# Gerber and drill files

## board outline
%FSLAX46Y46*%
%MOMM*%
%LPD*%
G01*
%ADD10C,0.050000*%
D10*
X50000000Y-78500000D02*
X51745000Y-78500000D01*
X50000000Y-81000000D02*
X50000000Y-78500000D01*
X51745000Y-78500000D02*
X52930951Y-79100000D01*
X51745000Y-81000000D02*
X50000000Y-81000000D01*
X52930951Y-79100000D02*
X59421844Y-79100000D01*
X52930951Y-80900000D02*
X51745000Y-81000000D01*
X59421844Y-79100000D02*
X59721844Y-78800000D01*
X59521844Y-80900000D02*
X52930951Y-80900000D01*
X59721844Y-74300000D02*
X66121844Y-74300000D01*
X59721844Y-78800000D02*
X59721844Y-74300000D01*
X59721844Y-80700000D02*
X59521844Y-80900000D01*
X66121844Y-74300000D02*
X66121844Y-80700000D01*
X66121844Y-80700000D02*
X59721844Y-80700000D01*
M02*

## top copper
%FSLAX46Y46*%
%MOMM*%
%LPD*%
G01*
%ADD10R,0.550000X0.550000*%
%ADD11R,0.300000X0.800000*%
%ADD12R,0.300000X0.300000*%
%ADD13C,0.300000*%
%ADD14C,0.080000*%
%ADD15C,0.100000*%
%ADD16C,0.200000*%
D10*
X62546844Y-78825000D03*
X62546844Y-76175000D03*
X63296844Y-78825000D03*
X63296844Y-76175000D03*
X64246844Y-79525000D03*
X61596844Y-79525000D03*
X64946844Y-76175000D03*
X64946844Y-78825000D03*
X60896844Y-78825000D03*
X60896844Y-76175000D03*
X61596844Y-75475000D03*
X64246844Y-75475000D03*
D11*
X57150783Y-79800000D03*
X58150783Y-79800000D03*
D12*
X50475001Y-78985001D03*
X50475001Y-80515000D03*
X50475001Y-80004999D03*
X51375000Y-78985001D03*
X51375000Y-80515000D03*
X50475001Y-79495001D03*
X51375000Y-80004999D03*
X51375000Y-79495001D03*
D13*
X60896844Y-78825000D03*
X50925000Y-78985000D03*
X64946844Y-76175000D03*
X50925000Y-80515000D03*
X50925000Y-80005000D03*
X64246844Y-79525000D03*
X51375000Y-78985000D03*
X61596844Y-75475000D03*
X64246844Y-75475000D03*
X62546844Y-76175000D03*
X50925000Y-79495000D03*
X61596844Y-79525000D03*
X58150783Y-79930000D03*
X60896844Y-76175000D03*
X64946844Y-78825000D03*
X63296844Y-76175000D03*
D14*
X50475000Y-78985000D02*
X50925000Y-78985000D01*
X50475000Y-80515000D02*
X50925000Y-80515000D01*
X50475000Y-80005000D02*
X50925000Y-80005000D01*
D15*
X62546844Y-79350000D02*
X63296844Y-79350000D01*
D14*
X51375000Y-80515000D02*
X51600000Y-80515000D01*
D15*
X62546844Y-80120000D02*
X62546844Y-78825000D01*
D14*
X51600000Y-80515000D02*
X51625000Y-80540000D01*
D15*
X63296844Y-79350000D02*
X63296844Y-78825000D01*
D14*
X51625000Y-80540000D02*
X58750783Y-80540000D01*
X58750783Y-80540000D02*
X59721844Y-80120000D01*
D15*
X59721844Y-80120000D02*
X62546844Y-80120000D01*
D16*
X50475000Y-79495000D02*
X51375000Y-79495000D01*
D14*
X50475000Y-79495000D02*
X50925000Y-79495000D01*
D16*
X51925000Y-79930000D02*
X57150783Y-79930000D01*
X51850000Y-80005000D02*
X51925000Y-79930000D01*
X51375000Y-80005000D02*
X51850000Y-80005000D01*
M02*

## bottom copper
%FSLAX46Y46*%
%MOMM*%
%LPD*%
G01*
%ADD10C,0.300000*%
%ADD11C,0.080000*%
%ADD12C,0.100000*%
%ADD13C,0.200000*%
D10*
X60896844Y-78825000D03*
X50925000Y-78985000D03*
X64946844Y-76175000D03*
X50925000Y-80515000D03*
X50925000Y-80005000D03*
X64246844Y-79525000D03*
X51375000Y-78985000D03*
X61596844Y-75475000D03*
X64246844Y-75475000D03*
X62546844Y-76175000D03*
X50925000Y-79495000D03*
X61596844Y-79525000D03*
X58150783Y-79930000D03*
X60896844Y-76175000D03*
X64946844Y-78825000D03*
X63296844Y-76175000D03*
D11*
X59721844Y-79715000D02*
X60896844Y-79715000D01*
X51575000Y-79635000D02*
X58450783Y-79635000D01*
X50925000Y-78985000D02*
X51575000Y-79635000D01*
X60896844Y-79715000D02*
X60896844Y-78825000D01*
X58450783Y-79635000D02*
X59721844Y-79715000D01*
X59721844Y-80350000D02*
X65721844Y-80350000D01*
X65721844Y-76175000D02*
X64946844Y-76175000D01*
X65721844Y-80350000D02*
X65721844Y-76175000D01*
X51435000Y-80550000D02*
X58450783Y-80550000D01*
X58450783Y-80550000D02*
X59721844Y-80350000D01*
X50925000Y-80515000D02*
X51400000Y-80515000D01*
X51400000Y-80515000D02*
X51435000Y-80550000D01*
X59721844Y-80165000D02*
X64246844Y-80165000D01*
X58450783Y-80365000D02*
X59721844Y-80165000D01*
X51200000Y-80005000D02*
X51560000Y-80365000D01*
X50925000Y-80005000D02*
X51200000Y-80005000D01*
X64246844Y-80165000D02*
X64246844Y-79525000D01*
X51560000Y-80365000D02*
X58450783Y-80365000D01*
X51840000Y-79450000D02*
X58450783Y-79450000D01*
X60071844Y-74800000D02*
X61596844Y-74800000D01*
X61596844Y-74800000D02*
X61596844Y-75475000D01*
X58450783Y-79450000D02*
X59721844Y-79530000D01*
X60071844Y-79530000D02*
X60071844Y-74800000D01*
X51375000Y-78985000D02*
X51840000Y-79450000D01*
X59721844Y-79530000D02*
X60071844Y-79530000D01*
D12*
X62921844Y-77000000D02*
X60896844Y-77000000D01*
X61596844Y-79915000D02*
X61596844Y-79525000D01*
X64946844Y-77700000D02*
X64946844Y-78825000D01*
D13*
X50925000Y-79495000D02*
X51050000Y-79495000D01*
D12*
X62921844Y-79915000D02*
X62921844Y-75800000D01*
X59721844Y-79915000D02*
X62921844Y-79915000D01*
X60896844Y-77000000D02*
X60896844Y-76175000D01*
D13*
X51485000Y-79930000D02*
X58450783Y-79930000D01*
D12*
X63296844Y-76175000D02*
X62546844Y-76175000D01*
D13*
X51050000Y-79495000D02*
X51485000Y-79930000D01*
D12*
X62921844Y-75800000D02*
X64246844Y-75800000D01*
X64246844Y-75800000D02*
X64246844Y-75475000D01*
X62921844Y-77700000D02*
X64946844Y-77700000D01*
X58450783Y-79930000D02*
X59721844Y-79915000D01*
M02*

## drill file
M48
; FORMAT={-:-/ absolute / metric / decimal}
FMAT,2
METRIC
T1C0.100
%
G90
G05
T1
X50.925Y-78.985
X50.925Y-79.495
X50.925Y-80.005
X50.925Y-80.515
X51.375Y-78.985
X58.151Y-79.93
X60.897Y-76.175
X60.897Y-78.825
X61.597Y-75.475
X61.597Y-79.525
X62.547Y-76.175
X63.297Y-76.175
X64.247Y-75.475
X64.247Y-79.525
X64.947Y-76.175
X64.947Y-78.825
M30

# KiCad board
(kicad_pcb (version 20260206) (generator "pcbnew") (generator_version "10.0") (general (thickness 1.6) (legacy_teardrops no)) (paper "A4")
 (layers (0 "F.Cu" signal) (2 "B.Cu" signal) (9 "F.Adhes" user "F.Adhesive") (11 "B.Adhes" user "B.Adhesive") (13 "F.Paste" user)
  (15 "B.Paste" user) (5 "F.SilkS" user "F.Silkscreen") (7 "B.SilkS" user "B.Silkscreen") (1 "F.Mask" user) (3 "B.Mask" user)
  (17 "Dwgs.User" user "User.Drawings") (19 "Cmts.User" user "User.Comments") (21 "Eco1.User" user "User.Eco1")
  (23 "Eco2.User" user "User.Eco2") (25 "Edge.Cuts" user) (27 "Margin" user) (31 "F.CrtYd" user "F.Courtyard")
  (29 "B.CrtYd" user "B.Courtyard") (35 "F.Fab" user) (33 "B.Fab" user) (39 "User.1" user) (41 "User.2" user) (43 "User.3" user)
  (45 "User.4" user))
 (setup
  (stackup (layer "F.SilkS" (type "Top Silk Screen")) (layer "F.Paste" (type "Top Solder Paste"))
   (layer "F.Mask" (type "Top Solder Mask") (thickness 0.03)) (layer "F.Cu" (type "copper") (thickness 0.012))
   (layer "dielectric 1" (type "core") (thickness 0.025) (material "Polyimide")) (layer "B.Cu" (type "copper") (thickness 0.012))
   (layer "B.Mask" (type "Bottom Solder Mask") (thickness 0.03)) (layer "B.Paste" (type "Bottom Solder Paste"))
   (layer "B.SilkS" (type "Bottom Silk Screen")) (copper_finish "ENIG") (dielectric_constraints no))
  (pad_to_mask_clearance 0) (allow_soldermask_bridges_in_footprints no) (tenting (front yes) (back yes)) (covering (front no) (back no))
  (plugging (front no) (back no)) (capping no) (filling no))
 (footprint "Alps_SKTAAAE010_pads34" (layer "F.Cu") (at 60.521844 77.5 90)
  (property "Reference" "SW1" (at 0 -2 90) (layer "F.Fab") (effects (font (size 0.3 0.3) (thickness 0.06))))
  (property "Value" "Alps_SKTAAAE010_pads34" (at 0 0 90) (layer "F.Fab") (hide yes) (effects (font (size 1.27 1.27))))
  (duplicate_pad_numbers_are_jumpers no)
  (pad "3" smd rect (at -1.325 0.375 90) (size 0.55 0.55) (layers "F.Cu" "F.Mask") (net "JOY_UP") (solder_mask_margin 0.05)
   (thermal_bridge_angle 45))
  (pad "4" smd rect (at 1.325 0.375 90) (size 0.55 0.55) (layers "F.Cu" "F.Mask") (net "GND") (solder_mask_margin 0.05)
   (thermal_bridge_angle 45)))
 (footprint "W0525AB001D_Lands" (layer "F.Cu") (at 57.650783 79.93)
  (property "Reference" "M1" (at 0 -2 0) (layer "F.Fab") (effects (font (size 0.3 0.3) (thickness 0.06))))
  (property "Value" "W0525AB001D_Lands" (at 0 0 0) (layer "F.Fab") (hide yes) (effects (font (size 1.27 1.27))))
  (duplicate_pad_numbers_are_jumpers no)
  (pad "1" smd rect (at -0.5 -0.13) (size 0.3 0.8) (layers "F.Cu" "F.Mask") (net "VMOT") (solder_mask_margin 0.05) (thermal_bridge_angle 45))
  (pad "2" smd rect (at 0.5 -0.13) (size 0.3 0.8) (layers "F.Cu" "F.Mask") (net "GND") (solder_mask_margin 0.05) (thermal_bridge_angle 45)))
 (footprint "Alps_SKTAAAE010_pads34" (layer "F.Cu") (at 62.921844 79.9 180)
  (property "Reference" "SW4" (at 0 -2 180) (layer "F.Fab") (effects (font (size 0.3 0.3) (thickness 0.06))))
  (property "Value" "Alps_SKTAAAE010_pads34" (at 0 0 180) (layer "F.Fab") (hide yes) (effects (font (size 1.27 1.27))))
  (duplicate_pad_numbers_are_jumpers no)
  (pad "3" smd rect (at -1.325 0.375 180) (size 0.55 0.55) (layers "F.Cu" "F.Mask") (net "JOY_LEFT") (solder_mask_margin 0.05)
   (thermal_bridge_angle 45))
  (pad "4" smd rect (at 1.325 0.375 180) (size 0.55 0.55) (layers "F.Cu" "F.Mask") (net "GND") (solder_mask_margin 0.05)
   (thermal_bridge_angle 45)))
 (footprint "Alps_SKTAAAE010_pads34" (layer "F.Cu") (at 62.921844 75.1)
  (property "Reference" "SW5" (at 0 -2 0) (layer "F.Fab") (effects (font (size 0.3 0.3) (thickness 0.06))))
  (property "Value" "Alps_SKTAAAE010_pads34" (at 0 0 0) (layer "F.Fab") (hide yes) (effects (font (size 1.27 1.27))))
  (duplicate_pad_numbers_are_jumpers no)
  (pad "3" smd rect (at -1.325 0.375) (size 0.55 0.55) (layers "F.Cu" "F.Mask") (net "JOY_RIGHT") (solder_mask_margin 0.05)
   (thermal_bridge_angle 45))
  (pad "4" smd rect (at 1.325 0.375) (size 0.55 0.55) (layers "F.Cu" "F.Mask") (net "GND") (solder_mask_margin 0.05)
   (thermal_bridge_angle 45)))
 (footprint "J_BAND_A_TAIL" (layer "F.Cu") (at 50.9 79.75)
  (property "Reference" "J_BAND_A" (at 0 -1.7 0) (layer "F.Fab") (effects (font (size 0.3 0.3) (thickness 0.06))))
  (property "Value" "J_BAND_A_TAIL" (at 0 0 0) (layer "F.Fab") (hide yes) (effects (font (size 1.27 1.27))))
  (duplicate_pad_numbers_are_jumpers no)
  (pad "1" smd rect (at -0.424999 -0.764999) (size 0.3 0.3) (layers "F.Cu" "F.Mask") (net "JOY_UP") (solder_mask_margin 0.05)
   (thermal_bridge_angle 45))
  (pad "2" smd rect (at -0.424999 0.765) (size 0.3 0.3) (layers "F.Cu" "F.Mask") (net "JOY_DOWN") (solder_mask_margin 0.05)
   (thermal_bridge_angle 45))
  (pad "3" smd rect (at -0.424999 0.254999) (size 0.3 0.3) (layers "F.Cu" "F.Mask") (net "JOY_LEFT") (solder_mask_margin 0.05)
   (thermal_bridge_angle 45))
  (pad "4" smd rect (at 0.475 -0.764999) (size 0.3 0.3) (layers "F.Cu" "F.Mask") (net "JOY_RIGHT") (solder_mask_margin 0.05)
   (thermal_bridge_angle 45))
  (pad "5" smd rect (at 0.475 0.765) (size 0.3 0.3) (layers "F.Cu" "F.Mask") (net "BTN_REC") (solder_mask_margin 0.05)
   (thermal_bridge_angle 45))
  (pad "6" smd rect (at -0.424999 -0.254999) (size 0.3 0.3) (layers "F.Cu" "F.Mask") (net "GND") (solder_mask_margin 0.05)
   (thermal_bridge_angle 45))
  (pad "7" smd rect (at 0.475 0.254999) (size 0.3 0.3) (layers "F.Cu" "F.Mask") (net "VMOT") (solder_mask_margin 0.05)
   (thermal_bridge_angle 45))
  (pad "8" smd rect (at 0.475 -0.254999) (size 0.3 0.3) (layers "F.Cu" "F.Mask") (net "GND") (solder_mask_margin 0.05)
   (thermal_bridge_angle 45)))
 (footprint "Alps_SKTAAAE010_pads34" (layer "F.Cu") (at 65.321844 77.5 -90)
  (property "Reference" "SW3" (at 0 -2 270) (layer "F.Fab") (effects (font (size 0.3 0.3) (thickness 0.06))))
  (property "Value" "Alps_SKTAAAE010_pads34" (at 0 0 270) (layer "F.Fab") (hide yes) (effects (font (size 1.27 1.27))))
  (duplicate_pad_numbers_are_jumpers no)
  (pad "3" smd rect (at -1.325 0.375 270) (size 0.55 0.55) (layers "F.Cu" "F.Mask") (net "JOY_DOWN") (solder_mask_margin 0.05)
   (thermal_bridge_angle 45))
  (pad "4" smd rect (at 1.325 0.375 270) (size 0.55 0.55) (layers "F.Cu" "F.Mask") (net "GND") (solder_mask_margin 0.05)
   (thermal_bridge_angle 45)))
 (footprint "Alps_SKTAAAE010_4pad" (layer "F.Cu") (at 62.921844 77.5 90)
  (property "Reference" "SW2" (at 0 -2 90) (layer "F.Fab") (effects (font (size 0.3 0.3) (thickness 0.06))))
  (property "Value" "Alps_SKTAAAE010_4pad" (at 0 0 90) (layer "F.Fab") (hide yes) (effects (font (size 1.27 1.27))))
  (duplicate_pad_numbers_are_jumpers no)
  (pad "1" smd rect (at -1.325 -0.375 90) (size 0.55 0.55) (layers "F.Cu" "F.Mask") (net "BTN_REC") (solder_mask_margin 0.05)
   (thermal_bridge_angle 45))
  (pad "2" smd rect (at 1.325 -0.375 90) (size 0.55 0.55) (layers "F.Cu" "F.Mask") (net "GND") (solder_mask_margin 0.05)
   (thermal_bridge_angle 45))
  (pad "3" smd rect (at -1.325 0.375 90) (size 0.55 0.55) (layers "F.Cu" "F.Mask") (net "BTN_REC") (solder_mask_margin 0.05)
   (thermal_bridge_angle 45))
  (pad "4" smd rect (at 1.325 0.375 90) (size 0.55 0.55) (layers "F.Cu" "F.Mask") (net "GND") (solder_mask_margin 0.05)
   (thermal_bridge_angle 45)))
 (gr_line (start 50 78.5) (end 51.745 78.5) (stroke (width 0.05) (type default)) (layer "Edge.Cuts"))
 (gr_line (start 50 81) (end 50 78.5) (stroke (width 0.05) (type default)) (layer "Edge.Cuts"))
 (gr_line (start 51.745 78.5) (end 52.930951 79.1) (stroke (width 0.05) (type default)) (layer "Edge.Cuts"))
 (gr_line (start 51.745 81) (end 50 81) (stroke (width 0.05) (type default)) (layer "Edge.Cuts"))
 (gr_line (start 52.930951 79.1) (end 59.421844 79.1) (stroke (width 0.05) (type default)) (layer "Edge.Cuts"))
 (gr_line (start 52.930951 80.9) (end 51.745 81) (stroke (width 0.05) (type default)) (layer "Edge.Cuts"))
 (gr_line (start 59.421844 79.1) (end 59.721844 78.8) (stroke (width 0.05) (type default)) (layer "Edge.Cuts"))
 (gr_line (start 59.521844 80.9) (end 52.930951 80.9) (stroke (width 0.05) (type default)) (layer "Edge.Cuts"))
 (gr_line (start 59.721844 74.3) (end 66.121844 74.3) (stroke (width 0.05) (type default)) (layer "Edge.Cuts"))
 (gr_line (start 59.721844 78.8) (end 59.721844 74.3) (stroke (width 0.05) (type default)) (layer "Edge.Cuts"))
 (gr_line (start 59.721844 80.7) (end 59.521844 80.9) (stroke (width 0.05) (type default)) (layer "Edge.Cuts"))
 (gr_line (start 66.121844 74.3) (end 66.121844 80.7) (stroke (width 0.05) (type default)) (layer "Edge.Cuts"))
 (gr_line (start 66.121844 80.7) (end 59.721844 80.7) (stroke (width 0.05) (type default)) (layer "Edge.Cuts"))
 (segment (start 50.475 78.985) (end 50.925 78.985) (width 0.08) (layer "F.Cu") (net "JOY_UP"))
 (via (at 60.896844 78.825) (size 0.3) (drill 0.1) (layers "F.Cu" "B.Cu") (tenting (front yes) (back yes)) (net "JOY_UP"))
 (via (at 50.925 78.985) (size 0.3) (drill 0.1) (layers "F.Cu" "B.Cu") (tenting (front yes) (back yes)) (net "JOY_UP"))
 (segment (start 51.575 79.635) (end 58.450783 79.635) (width 0.08) (layer "B.Cu") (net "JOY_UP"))
 (segment (start 59.721844 79.715) (end 60.896844 79.715) (width 0.08) (layer "B.Cu") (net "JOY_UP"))
 (segment (start 50.925 78.985) (end 51.575 79.635) (width 0.08) (layer "B.Cu") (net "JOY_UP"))
 (segment (start 60.896844 79.715) (end 60.896844 78.825) (width 0.08) (layer "B.Cu") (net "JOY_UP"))
 (segment (start 58.450783 79.635) (end 59.721844 79.715) (width 0.08) (layer "B.Cu") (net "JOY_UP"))
 (segment (start 50.475 80.515) (end 50.925 80.515) (width 0.08) (layer "F.Cu") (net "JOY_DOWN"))
 (via (at 50.925 80.515) (size 0.3) (drill 0.1) (layers "F.Cu" "B.Cu") (tenting (front yes) (back yes)) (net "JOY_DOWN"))
 (via (at 64.946844 76.175) (size 0.3) (drill 0.1) (layers "F.Cu" "B.Cu") (tenting (front yes) (back yes)) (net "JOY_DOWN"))
 (segment (start 50.925 80.515) (end 51.4 80.515) (width 0.08) (layer "B.Cu") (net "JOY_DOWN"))
 (segment (start 58.450783 80.55) (end 59.721844 80.35) (width 0.08) (layer "B.Cu") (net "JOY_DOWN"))
 (segment (start 59.721844 80.35) (end 65.721844 80.35) (width 0.08) (layer "B.Cu") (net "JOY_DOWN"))
 (segment (start 51.4 80.515) (end 51.435 80.55) (width 0.08) (layer "B.Cu") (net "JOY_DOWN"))
 (segment (start 51.435 80.55) (end 58.450783 80.55) (width 0.08) (layer "B.Cu") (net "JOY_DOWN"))
 (segment (start 65.721844 76.175) (end 64.946844 76.175) (width 0.08) (layer "B.Cu") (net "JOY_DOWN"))
 (segment (start 65.721844 80.35) (end 65.721844 76.175) (width 0.08) (layer "B.Cu") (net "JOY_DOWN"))
 (segment (start 50.475 80.005) (end 50.925 80.005) (width 0.08) (layer "F.Cu") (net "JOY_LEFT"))
 (via (at 50.925 80.005) (size 0.3) (drill 0.1) (layers "F.Cu" "B.Cu") (tenting (front yes) (back yes)) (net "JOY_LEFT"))
 (via (at 64.246844 79.525) (size 0.3) (drill 0.1) (layers "F.Cu" "B.Cu") (tenting (front yes) (back yes)) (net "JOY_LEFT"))
 (segment (start 51.2 80.005) (end 51.56 80.365) (width 0.08) (layer "B.Cu") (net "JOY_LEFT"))
 (segment (start 51.56 80.365) (end 58.450783 80.365) (width 0.08) (layer "B.Cu") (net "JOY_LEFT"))
 (segment (start 50.925 80.005) (end 51.2 80.005) (width 0.08) (layer "B.Cu") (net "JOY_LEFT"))
 (segment (start 58.450783 80.365) (end 59.721844 80.165) (width 0.08) (layer "B.Cu") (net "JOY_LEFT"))
 (segment (start 64.246844 80.165) (end 64.246844 79.525) (width 0.08) (layer "B.Cu") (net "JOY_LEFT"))
 (segment (start 59.721844 80.165) (end 64.246844 80.165) (width 0.08) (layer "B.Cu") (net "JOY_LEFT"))
 (via (at 61.596844 75.475) (size 0.3) (drill 0.1) (layers "F.Cu" "B.Cu") (tenting (front yes) (back yes)) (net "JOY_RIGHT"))
 (via (at 51.375 78.985) (size 0.3) (drill 0.1) (layers "F.Cu" "B.Cu") (tenting (front yes) (back yes)) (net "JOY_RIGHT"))
 (segment (start 61.596844 74.8) (end 61.596844 75.475) (width 0.08) (layer "B.Cu") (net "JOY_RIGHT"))
 (segment (start 58.450783 79.45) (end 59.721844 79.53) (width 0.08) (layer "B.Cu") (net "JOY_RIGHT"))
 (segment (start 60.071844 79.53) (end 60.071844 74.8) (width 0.08) (layer "B.Cu") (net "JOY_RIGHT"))
 (segment (start 59.721844 79.53) (end 60.071844 79.53) (width 0.08) (layer "B.Cu") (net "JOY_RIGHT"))
 (segment (start 51.375 78.985) (end 51.84 79.45) (width 0.08) (layer "B.Cu") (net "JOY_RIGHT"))
 (segment (start 51.84 79.45) (end 58.450783 79.45) (width 0.08) (layer "B.Cu") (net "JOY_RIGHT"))
 (segment (start 60.071844 74.8) (end 61.596844 74.8) (width 0.08) (layer "B.Cu") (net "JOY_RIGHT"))
 (segment (start 51.6 80.515) (end 51.625 80.54) (width 0.08) (layer "F.Cu") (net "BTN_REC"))
 (segment (start 62.546844 79.35) (end 63.296844 79.35) (width 0.1) (layer "F.Cu") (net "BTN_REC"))
 (segment (start 63.296844 79.35) (end 63.296844 78.825) (width 0.1) (layer "F.Cu") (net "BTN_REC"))
 (segment (start 62.546844 80.12) (end 62.546844 78.825) (width 0.1) (layer "F.Cu") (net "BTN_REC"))
 (segment (start 58.750783 80.54) (end 59.721844 80.12) (width 0.08) (layer "F.Cu") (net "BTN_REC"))
 (segment (start 51.375 80.515) (end 51.6 80.515) (width 0.08) (layer "F.Cu") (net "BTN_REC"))
 (segment (start 51.625 80.54) (end 58.750783 80.54) (width 0.08) (layer "F.Cu") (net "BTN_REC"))
 (segment (start 59.721844 80.12) (end 62.546844 80.12) (width 0.1) (layer "F.Cu") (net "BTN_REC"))
 (segment (start 50.475 79.495) (end 50.925 79.495) (width 0.08) (layer "F.Cu") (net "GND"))
 (segment (start 50.475 79.495) (end 51.375 79.495) (width 0.2) (layer "F.Cu") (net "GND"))
 (via (at 64.946844 78.825) (size 0.3) (drill 0.1) (layers "F.Cu" "B.Cu") (tenting (front yes) (back yes)) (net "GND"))
 (via (at 50.925 79.495) (size 0.3) (drill 0.1) (layers "F.Cu" "B.Cu") (tenting (front yes) (back yes)) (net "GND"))
 (via (at 63.296844 76.175) (size 0.3) (drill 0.1) (layers "F.Cu" "B.Cu") (tenting (front yes) (back yes)) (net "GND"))
 (via (at 60.896844 76.175) (size 0.3) (drill 0.1) (layers "F.Cu" "B.Cu") (tenting (front yes) (back yes)) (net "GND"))
 (via (at 61.596844 79.525) (size 0.3) (drill 0.1) (layers "F.Cu" "B.Cu") (tenting (front yes) (back yes)) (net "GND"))
 (via (at 64.246844 75.475) (size 0.3) (drill 0.1) (layers "F.Cu" "B.Cu") (tenting (front yes) (back yes)) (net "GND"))
 (via (at 62.546844 76.175) (size 0.3) (drill 0.1) (layers "F.Cu" "B.Cu") (tenting (front yes) (back yes)) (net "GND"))
 (via (at 58.150783 79.93) (size 0.3) (drill 0.1) (layers "F.Cu" "B.Cu") (tenting (front yes) (back yes)) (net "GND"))
 (segment (start 59.721844 79.915) (end 62.921844 79.915) (width 0.1) (layer "B.Cu") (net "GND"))
 (segment (start 62.921844 77) (end 60.896844 77) (width 0.1) (layer "B.Cu") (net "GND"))
 (segment (start 64.946844 77.7) (end 64.946844 78.825) (width 0.1) (layer "B.Cu") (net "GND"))
 (segment (start 62.921844 79.915) (end 62.921844 75.8) (width 0.1) (layer "B.Cu") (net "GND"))
 (segment (start 50.925 79.495) (end 51.05 79.495) (width 0.2) (layer "B.Cu") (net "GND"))
 (segment (start 51.485 79.93) (end 58.450783 79.93) (width 0.2) (layer "B.Cu") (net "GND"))
 (segment (start 62.921844 75.8) (end 64.246844 75.8) (width 0.1) (layer "B.Cu") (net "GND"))
 (segment (start 58.450783 79.93) (end 59.721844 79.915) (width 0.1) (layer "B.Cu") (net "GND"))
 (segment (start 61.596844 79.915) (end 61.596844 79.525) (width 0.1) (layer "B.Cu") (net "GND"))
 (segment (start 64.246844 75.8) (end 64.246844 75.475) (width 0.1) (layer "B.Cu") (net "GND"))
 (segment (start 63.296844 76.175) (end 62.546844 76.175) (width 0.1) (layer "B.Cu") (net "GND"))
 (segment (start 62.921844 77.7) (end 64.946844 77.7) (width 0.1) (layer "B.Cu") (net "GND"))
 (segment (start 51.05 79.495) (end 51.485 79.93) (width 0.2) (layer "B.Cu") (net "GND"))
 (segment (start 60.896844 77) (end 60.896844 76.175) (width 0.1) (layer "B.Cu") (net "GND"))
 (segment (start 51.925 79.93) (end 57.150783 79.93) (width 0.2) (layer "F.Cu") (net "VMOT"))
 (segment (start 51.375 80.005) (end 51.85 80.005) (width 0.2) (layer "F.Cu") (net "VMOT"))
 (segment (start 51.85 80.005) (end 51.925 79.93) (width 0.2) (layer "F.Cu") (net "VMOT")))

